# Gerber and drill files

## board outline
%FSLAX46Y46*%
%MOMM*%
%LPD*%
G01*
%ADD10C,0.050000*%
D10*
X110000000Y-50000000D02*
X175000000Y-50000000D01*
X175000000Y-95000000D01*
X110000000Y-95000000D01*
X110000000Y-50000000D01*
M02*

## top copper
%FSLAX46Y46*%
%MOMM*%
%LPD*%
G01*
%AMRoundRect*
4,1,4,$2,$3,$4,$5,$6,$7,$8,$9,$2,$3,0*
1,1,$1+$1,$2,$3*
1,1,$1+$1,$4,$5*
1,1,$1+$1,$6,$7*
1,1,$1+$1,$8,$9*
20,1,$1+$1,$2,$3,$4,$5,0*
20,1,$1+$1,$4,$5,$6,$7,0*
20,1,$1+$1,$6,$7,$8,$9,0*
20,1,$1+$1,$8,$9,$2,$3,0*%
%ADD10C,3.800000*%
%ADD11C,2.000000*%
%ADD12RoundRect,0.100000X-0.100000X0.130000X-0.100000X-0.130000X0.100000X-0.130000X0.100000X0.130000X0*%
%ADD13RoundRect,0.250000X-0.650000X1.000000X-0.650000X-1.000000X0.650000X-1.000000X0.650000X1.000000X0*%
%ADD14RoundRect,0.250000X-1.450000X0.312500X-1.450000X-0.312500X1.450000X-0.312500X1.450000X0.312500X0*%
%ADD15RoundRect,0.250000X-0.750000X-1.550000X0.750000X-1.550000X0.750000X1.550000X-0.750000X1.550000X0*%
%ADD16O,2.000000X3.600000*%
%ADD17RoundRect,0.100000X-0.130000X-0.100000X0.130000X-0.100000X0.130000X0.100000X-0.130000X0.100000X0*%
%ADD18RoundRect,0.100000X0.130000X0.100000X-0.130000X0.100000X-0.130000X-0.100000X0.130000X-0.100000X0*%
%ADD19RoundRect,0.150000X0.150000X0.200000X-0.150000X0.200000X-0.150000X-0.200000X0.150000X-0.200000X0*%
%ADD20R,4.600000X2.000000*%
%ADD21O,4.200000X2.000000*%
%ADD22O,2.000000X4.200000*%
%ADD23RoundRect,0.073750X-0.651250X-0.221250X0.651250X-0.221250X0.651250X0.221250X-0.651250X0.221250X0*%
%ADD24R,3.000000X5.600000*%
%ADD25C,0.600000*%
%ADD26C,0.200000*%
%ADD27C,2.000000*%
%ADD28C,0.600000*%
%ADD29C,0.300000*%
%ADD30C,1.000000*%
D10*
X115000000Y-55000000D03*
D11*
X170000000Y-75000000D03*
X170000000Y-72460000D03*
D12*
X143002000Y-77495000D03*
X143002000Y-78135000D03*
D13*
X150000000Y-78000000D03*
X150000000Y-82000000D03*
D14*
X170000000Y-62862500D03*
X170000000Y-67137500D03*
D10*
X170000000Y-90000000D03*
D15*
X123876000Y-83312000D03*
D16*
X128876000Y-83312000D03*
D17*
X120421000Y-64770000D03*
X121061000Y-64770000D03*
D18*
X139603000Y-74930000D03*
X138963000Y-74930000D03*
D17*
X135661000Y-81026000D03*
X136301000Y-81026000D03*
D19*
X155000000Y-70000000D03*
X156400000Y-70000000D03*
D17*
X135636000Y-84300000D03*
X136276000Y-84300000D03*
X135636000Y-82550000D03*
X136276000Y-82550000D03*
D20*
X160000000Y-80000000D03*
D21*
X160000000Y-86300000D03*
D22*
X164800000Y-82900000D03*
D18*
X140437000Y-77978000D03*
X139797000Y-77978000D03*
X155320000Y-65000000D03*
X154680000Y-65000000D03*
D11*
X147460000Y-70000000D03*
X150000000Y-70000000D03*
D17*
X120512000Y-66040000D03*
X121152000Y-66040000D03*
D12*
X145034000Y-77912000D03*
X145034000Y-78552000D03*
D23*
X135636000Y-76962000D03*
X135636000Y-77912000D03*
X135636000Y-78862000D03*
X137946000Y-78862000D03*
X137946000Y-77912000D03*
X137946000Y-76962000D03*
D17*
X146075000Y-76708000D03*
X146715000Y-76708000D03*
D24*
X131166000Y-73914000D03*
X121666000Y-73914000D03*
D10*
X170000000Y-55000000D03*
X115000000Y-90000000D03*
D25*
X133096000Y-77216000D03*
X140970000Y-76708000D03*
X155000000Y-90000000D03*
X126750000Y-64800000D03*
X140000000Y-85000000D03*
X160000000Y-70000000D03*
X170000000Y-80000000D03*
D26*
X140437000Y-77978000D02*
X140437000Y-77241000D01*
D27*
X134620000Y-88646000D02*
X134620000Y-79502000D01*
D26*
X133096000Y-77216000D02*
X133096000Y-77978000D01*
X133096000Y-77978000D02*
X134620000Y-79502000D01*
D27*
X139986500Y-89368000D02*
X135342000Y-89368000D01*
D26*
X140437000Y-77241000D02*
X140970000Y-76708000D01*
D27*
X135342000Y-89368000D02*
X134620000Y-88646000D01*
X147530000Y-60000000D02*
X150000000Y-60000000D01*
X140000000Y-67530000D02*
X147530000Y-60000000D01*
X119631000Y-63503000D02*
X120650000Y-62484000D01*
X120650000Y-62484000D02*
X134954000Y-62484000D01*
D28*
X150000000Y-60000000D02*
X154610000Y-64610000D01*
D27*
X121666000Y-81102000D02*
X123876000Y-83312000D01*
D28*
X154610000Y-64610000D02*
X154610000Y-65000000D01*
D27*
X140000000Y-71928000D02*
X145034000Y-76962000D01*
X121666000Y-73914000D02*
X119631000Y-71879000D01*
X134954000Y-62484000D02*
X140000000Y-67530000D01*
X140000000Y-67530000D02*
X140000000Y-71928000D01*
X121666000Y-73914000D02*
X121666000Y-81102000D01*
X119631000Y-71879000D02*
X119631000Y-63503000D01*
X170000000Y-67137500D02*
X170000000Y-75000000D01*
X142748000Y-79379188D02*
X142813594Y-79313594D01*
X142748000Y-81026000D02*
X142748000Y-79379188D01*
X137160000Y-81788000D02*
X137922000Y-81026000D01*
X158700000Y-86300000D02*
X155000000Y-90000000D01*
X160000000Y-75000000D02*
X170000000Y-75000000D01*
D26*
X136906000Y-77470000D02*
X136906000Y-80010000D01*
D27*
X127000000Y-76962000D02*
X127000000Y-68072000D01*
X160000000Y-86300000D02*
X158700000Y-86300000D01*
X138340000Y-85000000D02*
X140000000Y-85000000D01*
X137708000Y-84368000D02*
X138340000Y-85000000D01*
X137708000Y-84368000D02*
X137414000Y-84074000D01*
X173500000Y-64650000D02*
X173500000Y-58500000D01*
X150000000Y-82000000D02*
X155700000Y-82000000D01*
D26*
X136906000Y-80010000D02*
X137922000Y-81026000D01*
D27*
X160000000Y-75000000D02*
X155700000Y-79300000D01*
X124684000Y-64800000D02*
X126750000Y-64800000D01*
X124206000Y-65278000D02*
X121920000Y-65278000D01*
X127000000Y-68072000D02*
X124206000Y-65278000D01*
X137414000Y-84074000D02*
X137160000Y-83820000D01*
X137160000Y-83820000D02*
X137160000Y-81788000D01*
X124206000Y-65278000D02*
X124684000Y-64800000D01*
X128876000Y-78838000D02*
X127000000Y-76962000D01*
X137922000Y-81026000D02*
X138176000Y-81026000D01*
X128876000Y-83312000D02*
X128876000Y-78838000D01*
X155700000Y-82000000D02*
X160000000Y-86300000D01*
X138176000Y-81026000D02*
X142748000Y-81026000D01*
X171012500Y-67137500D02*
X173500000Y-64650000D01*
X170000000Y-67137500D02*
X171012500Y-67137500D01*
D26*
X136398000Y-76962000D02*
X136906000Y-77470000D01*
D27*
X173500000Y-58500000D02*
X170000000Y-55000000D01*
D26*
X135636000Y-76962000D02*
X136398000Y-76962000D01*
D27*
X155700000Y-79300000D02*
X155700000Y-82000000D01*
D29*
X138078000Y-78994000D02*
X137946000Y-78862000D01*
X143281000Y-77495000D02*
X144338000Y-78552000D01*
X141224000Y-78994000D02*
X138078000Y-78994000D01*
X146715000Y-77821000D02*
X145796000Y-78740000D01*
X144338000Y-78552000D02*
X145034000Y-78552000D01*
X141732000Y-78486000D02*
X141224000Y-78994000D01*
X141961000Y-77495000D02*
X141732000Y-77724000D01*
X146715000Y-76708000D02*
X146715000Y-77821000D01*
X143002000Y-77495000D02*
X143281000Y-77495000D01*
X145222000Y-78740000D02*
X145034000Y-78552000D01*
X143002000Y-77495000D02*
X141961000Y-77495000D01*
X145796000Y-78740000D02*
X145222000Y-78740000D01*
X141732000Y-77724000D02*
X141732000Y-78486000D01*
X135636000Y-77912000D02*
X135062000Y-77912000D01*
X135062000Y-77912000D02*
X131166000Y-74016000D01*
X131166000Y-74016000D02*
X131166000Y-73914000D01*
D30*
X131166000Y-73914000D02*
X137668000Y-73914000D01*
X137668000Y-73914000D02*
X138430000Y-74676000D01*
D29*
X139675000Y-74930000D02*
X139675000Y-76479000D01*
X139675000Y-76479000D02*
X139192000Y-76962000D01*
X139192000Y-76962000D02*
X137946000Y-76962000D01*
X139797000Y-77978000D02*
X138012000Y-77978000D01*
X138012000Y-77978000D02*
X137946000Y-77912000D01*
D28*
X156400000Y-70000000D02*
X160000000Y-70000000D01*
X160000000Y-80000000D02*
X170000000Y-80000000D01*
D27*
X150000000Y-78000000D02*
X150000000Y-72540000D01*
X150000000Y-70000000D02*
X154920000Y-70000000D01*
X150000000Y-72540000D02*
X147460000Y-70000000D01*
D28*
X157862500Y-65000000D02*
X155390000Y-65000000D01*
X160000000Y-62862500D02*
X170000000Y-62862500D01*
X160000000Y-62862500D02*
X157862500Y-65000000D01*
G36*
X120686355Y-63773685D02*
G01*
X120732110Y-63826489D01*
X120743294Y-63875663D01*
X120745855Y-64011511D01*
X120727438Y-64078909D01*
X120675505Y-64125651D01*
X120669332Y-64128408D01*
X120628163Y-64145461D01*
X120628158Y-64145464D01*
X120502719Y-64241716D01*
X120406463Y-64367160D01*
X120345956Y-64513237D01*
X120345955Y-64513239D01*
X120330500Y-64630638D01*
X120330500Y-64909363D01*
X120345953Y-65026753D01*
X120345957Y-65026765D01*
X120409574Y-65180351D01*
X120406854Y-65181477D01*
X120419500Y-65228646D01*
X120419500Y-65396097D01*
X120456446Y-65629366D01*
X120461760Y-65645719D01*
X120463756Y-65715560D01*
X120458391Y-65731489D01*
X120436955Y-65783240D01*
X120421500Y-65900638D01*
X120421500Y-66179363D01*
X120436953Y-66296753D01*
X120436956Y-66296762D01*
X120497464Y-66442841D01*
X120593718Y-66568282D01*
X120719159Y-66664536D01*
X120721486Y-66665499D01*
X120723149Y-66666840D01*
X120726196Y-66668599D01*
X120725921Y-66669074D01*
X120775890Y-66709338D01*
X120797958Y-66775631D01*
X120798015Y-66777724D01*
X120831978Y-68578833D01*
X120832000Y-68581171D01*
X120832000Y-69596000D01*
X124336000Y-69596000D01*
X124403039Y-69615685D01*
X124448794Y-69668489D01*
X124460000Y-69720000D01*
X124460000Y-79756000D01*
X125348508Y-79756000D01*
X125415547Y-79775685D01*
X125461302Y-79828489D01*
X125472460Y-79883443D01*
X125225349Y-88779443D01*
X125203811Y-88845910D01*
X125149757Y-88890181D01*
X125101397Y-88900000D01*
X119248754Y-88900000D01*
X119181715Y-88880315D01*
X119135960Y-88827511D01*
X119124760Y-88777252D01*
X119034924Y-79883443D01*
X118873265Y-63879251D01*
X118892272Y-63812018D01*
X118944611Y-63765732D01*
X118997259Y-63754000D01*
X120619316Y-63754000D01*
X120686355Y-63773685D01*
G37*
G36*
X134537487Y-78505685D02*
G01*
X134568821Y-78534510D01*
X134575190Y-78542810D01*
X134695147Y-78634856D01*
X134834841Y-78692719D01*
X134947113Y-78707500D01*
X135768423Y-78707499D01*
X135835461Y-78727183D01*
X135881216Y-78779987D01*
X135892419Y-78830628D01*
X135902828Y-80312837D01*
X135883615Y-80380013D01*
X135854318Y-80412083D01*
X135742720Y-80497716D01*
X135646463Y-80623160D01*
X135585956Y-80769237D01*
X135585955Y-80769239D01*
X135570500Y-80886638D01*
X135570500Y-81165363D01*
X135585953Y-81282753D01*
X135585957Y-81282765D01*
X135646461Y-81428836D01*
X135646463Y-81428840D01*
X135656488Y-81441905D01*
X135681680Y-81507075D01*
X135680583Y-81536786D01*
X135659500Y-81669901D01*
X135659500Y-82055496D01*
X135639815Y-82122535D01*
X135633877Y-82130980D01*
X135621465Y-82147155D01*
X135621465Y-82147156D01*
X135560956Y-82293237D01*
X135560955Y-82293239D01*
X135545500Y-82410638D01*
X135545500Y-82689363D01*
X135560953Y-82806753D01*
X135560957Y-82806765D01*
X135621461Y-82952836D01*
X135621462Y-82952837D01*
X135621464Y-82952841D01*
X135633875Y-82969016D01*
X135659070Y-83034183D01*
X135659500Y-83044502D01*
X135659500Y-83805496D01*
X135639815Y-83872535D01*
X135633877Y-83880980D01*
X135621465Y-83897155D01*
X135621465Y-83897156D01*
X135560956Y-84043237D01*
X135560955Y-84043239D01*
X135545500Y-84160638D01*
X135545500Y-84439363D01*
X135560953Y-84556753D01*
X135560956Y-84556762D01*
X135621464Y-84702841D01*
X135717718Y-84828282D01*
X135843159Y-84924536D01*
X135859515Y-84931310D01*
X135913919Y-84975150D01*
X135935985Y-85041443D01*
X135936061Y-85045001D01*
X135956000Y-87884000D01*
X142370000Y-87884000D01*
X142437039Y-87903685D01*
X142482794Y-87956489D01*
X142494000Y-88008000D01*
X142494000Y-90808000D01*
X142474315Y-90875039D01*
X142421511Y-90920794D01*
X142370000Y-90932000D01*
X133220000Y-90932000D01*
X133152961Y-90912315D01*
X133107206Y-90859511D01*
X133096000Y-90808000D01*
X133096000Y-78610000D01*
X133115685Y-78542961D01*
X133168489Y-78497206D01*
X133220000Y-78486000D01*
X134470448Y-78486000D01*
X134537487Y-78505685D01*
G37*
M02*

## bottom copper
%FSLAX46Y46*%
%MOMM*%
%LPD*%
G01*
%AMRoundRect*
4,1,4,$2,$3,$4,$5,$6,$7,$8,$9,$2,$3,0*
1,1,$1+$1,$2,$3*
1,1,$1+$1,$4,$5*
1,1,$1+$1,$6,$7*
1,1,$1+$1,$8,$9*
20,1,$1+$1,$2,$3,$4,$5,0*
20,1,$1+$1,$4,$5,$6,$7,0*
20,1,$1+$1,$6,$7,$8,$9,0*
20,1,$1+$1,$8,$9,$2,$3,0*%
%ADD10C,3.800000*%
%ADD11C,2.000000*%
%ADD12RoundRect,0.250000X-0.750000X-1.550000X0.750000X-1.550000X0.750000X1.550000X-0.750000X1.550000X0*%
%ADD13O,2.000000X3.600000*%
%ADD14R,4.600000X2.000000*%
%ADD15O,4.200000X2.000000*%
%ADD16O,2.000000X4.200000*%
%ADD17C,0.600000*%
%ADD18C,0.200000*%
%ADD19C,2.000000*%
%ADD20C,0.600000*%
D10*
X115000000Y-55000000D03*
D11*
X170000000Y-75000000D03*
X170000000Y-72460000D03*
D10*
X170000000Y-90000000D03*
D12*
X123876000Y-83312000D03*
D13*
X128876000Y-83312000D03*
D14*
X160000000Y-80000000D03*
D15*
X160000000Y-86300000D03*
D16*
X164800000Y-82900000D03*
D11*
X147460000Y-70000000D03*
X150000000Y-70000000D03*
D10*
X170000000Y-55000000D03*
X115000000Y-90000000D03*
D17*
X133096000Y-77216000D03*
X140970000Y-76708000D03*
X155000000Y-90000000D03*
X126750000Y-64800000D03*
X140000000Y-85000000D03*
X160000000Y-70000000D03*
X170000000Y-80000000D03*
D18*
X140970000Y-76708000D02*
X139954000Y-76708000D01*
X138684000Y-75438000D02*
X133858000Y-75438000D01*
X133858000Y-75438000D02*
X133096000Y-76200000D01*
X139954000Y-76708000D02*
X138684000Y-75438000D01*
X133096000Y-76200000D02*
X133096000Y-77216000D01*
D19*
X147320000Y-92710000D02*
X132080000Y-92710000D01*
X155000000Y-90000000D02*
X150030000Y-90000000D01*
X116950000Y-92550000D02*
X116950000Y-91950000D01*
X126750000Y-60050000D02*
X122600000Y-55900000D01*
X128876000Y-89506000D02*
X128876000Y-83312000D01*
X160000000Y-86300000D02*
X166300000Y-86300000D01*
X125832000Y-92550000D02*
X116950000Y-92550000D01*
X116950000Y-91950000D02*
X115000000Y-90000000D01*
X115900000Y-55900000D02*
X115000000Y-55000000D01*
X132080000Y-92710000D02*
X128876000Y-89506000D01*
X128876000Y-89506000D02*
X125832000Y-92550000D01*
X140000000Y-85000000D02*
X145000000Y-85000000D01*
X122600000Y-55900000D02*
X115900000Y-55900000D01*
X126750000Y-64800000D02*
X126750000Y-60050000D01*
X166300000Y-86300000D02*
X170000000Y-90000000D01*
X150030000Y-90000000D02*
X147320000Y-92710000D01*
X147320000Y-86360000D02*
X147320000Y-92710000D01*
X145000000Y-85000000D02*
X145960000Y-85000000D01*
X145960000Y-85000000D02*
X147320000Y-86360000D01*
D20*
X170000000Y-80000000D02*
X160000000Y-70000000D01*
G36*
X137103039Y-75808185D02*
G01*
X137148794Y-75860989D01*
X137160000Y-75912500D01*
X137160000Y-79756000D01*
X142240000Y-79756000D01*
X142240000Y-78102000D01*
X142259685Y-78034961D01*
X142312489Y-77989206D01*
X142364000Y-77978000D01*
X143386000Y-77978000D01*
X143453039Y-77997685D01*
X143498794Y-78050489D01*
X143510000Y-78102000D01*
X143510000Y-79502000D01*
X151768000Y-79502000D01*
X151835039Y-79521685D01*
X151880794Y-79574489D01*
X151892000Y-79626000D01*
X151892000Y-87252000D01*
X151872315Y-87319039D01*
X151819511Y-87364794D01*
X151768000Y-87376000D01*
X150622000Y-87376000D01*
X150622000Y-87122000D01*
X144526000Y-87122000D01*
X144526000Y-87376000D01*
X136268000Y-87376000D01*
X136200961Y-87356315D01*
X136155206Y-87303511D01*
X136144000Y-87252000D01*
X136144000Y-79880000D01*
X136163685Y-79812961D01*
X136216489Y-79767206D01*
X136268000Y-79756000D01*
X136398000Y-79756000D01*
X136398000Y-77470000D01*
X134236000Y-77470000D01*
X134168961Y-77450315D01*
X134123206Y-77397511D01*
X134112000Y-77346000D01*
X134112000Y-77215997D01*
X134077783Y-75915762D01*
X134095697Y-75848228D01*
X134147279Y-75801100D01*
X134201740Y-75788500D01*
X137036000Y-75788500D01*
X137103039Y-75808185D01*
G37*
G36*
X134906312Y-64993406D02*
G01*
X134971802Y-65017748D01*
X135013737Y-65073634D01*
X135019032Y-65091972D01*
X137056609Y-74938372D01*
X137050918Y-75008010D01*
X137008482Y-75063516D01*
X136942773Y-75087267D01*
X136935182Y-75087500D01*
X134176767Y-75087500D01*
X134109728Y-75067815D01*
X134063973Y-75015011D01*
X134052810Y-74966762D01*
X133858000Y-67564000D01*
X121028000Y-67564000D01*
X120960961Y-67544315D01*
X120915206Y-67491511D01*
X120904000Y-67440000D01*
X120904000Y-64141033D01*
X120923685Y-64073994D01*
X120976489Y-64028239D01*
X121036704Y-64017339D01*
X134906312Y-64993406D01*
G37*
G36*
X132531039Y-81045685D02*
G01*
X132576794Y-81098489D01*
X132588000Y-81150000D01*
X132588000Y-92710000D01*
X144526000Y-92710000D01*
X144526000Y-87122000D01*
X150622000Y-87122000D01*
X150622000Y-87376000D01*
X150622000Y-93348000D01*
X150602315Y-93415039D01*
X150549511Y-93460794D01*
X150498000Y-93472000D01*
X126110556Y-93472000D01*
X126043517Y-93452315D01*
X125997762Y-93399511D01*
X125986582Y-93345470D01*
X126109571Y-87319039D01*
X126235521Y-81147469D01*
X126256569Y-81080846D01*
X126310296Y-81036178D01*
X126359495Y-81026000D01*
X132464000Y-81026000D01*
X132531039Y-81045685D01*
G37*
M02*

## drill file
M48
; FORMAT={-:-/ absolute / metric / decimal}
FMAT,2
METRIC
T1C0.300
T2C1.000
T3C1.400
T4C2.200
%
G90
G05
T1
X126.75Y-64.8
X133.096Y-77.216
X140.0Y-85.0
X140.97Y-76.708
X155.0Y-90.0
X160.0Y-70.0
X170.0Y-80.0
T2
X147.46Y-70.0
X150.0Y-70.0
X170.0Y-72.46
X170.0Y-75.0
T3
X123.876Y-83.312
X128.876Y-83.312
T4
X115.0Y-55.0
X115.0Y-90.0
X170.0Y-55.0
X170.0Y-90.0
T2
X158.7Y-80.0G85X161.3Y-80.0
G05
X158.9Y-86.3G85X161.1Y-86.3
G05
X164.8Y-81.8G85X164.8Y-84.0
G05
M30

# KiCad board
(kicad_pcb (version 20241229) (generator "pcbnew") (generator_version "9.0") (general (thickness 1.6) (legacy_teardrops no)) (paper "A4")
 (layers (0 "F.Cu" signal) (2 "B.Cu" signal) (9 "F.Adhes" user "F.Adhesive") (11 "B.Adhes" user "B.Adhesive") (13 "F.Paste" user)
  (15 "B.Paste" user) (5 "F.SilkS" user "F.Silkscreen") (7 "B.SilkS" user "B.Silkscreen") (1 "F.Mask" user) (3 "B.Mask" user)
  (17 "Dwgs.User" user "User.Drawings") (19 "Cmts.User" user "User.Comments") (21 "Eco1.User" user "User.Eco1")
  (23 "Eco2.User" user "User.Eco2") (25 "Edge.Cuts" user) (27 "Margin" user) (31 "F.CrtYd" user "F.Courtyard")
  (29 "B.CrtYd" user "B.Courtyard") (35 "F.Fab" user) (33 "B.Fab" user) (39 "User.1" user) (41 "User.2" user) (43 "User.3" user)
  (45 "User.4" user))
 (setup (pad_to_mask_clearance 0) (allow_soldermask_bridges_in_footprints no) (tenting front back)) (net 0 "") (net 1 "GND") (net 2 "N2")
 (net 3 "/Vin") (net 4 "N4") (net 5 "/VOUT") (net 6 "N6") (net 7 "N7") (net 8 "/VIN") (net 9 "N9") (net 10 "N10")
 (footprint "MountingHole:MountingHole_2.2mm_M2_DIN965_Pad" (layer "F.Cu") (at 115 55)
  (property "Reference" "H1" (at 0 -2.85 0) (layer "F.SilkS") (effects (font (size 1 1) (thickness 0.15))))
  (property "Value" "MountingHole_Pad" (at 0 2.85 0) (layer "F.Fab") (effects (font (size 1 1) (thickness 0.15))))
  (pad "1" thru_hole circle (at 0 0) (size 3.8 3.8) (drill 2.2) (layers "*.Cu" "*.Mask") (remove_unused_layers no) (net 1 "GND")
   (zone_connect 2)))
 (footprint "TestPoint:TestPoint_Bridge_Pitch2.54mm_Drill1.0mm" (layer "F.Cu") (at 170 75 90)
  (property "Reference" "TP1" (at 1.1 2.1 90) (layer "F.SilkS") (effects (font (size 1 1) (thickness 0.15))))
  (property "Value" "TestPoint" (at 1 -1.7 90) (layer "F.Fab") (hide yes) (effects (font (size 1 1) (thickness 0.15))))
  (pad "1" thru_hole circle (at 0 0 90) (size 2 2) (drill 1) (layers "*.Cu" "*.Mask") (remove_unused_layers no) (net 1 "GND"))
  (pad "1" thru_hole circle (at 2.54 0 90) (size 2 2) (drill 1) (layers "*.Cu" "*.Mask") (remove_unused_layers no) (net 1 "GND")))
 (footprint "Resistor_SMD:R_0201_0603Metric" (layer "F.Cu") (at 143.002 77.815 -90)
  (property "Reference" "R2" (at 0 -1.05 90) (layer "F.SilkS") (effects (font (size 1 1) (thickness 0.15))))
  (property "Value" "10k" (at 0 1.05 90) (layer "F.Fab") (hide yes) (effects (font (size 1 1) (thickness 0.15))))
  (pad "" smd roundrect (at -0.345 0 270) (size 0.318 0.36) (layers "F.Paste") (roundrect_rratio 0.25))
  (pad "" smd roundrect (at 0.345 0 270) (size 0.318 0.36) (layers "F.Paste") (roundrect_rratio 0.25))
  (pad "1" smd roundrect (at -0.32 0 270) (size 0.46 0.4) (layers "F.Cu" "F.Mask") (roundrect_rratio 0.25) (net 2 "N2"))
  (pad "2" smd roundrect (at 0.32 0 270) (size 0.46 0.4) (layers "F.Cu" "F.Mask") (roundrect_rratio 0.25) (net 1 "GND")))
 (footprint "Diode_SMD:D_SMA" (layer "F.Cu") (at 150 80 -90)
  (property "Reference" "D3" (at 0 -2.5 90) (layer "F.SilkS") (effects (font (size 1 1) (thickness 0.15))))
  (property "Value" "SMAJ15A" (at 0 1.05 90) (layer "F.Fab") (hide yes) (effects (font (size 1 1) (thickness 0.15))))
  (pad "1" smd roundrect (at -2 0 270) (size 2.5 1.8) (layers "F.Cu" "F.Mask" "F.Paste") (roundrect_rratio 0.1388888889) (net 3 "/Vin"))
  (pad "2" smd roundrect (at 2 0 270) (size 2.5 1.8) (layers "F.Cu" "F.Mask" "F.Paste") (roundrect_rratio 0.1388888889) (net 1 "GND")))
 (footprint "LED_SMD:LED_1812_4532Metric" (layer "F.Cu") (at 170 65 -90)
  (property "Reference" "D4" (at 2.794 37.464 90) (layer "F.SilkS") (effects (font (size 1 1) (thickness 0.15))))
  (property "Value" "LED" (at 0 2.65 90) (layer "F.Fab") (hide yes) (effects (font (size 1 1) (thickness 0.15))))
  (pad "1" smd roundrect (at -2.1375 0 270) (size 1.125 3.4) (layers "F.Cu" "F.Mask" "F.Paste") (roundrect_rratio 0.222222) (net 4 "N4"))
  (pad "2" smd roundrect (at 2.1375 0 270) (size 1.125 3.4) (layers "F.Cu" "F.Mask" "F.Paste") (roundrect_rratio 0.222222) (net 1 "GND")))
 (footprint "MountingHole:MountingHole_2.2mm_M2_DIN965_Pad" (layer "F.Cu") (at 170 90)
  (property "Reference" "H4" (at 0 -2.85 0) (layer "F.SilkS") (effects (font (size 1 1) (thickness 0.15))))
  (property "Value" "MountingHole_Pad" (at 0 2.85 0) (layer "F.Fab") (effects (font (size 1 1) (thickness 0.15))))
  (pad "1" thru_hole circle (at 0 0) (size 3.8 3.8) (drill 2.2) (layers "*.Cu" "*.Mask") (remove_unused_layers no) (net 1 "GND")
   (zone_connect 2)))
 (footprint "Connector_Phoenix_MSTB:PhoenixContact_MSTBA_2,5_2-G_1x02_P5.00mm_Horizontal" (layer "F.Cu") (at 123.876 83.312)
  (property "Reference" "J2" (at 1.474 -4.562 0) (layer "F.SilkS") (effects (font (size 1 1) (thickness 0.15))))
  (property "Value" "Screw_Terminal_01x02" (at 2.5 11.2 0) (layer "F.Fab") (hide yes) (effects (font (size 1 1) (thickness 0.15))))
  (pad "1" thru_hole roundrect (at 0 0) (size 2 3.6) (drill 1.4) (layers "*.Cu" "*.Mask") (remove_unused_layers no) (roundrect_rratio 0.125)
   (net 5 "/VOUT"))
  (pad "2" thru_hole oval (at 5 0) (size 2 3.6) (drill 1.4) (layers "*.Cu" "*.Mask") (remove_unused_layers no) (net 1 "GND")))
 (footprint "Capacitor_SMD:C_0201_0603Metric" (layer "F.Cu") (at 120.741 64.77)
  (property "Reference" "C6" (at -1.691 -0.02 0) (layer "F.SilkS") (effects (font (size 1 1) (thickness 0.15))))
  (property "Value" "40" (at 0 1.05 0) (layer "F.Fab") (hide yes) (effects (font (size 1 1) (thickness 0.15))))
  (pad "" smd roundrect (at -0.345 0) (size 0.318 0.36) (layers "F.Paste") (roundrect_rratio 0.25))
  (pad "" smd roundrect (at 0.345 0) (size 0.318 0.36) (layers "F.Paste") (roundrect_rratio 0.25))
  (pad "1" smd roundrect (at -0.32 0) (size 0.46 0.4) (layers "F.Cu" "F.Mask") (roundrect_rratio 0.25) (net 5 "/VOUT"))
  (pad "2" smd roundrect (at 0.32 0) (size 0.46 0.4) (layers "F.Cu" "F.Mask") (roundrect_rratio 0.25) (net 1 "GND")))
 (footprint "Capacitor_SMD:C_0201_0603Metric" (layer "F.Cu") (at 139.283 74.93 180)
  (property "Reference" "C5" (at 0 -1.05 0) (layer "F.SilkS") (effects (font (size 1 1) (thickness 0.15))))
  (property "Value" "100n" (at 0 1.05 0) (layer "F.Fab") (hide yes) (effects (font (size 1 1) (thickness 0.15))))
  (pad "" smd roundrect (at -0.345 0 180) (size 0.318 0.36) (layers "F.Paste") (roundrect_rratio 0.25))
  (pad "" smd roundrect (at 0.345 0 180) (size 0.318 0.36) (layers "F.Paste") (roundrect_rratio 0.25))
  (pad "1" smd roundrect (at -0.32 0 180) (size 0.46 0.4) (layers "F.Cu" "F.Mask") (roundrect_rratio 0.25) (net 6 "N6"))
  (pad "2" smd roundrect (at 0.32 0 180) (size 0.46 0.4) (layers "F.Cu" "F.Mask") (roundrect_rratio 0.25) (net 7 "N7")))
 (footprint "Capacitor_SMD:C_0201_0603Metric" (layer "F.Cu") (at 135.981 81.026)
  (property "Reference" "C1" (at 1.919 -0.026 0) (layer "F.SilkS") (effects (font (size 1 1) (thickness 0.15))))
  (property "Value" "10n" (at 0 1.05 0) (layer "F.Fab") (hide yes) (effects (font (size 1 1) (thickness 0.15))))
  (pad "" smd roundrect (at -0.345 0) (size 0.318 0.36) (layers "F.Paste") (roundrect_rratio 0.25))
  (pad "" smd roundrect (at 0.345 0) (size 0.318 0.36) (layers "F.Paste") (roundrect_rratio 0.25))
  (pad "1" smd roundrect (at -0.32 0) (size 0.46 0.4) (layers "F.Cu" "F.Mask") (roundrect_rratio 0.25) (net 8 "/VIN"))
  (pad "2" smd roundrect (at 0.32 0) (size 0.46 0.4) (layers "F.Cu" "F.Mask") (roundrect_rratio 0.25) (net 1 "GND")))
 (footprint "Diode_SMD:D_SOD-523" (layer "F.Cu") (at 155.7 70)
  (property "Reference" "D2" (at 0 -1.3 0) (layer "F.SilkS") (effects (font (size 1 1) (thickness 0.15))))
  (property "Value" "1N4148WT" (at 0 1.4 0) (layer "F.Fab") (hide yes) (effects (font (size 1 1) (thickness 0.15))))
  (pad "1" smd roundrect (at -0.7 0 180) (size 0.6 0.7) (layers "F.Cu" "F.Mask" "F.Paste") (roundrect_rratio 0.25) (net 3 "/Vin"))
  (pad "2" smd roundrect (at 0.7 0 180) (size 0.6 0.7) (layers "F.Cu" "F.Mask" "F.Paste") (roundrect_rratio 0.25) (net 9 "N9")))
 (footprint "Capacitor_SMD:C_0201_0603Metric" (layer "F.Cu") (at 135.956 84.3)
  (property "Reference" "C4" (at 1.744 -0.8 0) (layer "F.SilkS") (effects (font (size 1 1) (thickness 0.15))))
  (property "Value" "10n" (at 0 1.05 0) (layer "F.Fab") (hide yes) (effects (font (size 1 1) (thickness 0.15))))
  (pad "" smd roundrect (at -0.345 0) (size 0.318 0.36) (layers "F.Paste") (roundrect_rratio 0.25))
  (pad "" smd roundrect (at 0.345 0) (size 0.318 0.36) (layers "F.Paste") (roundrect_rratio 0.25))
  (pad "1" smd roundrect (at -0.32 0) (size 0.46 0.4) (layers "F.Cu" "F.Mask") (roundrect_rratio 0.25) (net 8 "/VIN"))
  (pad "2" smd roundrect (at 0.32 0) (size 0.46 0.4) (layers "F.Cu" "F.Mask") (roundrect_rratio 0.25) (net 1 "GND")))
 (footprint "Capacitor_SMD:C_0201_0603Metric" (layer "F.Cu") (at 135.956 82.55)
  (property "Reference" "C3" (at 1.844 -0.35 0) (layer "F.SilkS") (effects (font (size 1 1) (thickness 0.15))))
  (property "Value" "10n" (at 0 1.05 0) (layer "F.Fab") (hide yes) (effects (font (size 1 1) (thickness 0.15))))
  (pad "" smd roundrect (at -0.345 0) (size 0.318 0.36) (layers "F.Paste") (roundrect_rratio 0.25))
  (pad "" smd roundrect (at 0.345 0) (size 0.318 0.36) (layers "F.Paste") (roundrect_rratio 0.25))
  (pad "1" smd roundrect (at -0.32 0) (size 0.46 0.4) (layers "F.Cu" "F.Mask") (roundrect_rratio 0.25) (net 8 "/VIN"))
  (pad "2" smd roundrect (at 0.32 0) (size 0.46 0.4) (layers "F.Cu" "F.Mask") (roundrect_rratio 0.25) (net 1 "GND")))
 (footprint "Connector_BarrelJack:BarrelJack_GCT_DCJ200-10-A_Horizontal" (layer "F.Cu") (at 160 80)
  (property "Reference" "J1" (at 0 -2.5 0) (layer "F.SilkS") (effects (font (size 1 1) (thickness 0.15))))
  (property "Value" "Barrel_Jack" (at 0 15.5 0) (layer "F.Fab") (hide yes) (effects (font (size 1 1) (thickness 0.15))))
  (pad "1" thru_hole rect (at 0 0) (size 4.6 2) (drill oval 3.6 1) (layers "*.Cu" "*.Mask") (remove_unused_layers no) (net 9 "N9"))
  (pad "2" thru_hole oval (at 0 6.3) (size 4.2 2) (drill oval 3.2 1) (layers "*.Cu" "*.Mask") (remove_unused_layers no) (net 1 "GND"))
  (pad "3" thru_hole oval (at 4.8 2.9) (size 2 4.2) (drill oval 1 3.2) (layers "*.Cu" "*.Mask") (remove_unused_layers no)))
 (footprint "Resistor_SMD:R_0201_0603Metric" (layer "F.Cu") (at 140.117 77.978 180)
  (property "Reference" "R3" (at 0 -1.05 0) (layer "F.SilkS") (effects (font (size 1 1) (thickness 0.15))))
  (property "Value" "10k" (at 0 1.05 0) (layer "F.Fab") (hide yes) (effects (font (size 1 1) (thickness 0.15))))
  (pad "" smd roundrect (at -0.345 0 180) (size 0.318 0.36) (layers "F.Paste") (roundrect_rratio 0.25))
  (pad "" smd roundrect (at 0.345 0 180) (size 0.318 0.36) (layers "F.Paste") (roundrect_rratio 0.25))
  (pad "1" smd roundrect (at -0.32 0 180) (size 0.46 0.4) (layers "F.Cu" "F.Mask") (roundrect_rratio 0.25) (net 8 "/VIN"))
  (pad "2" smd roundrect (at 0.32 0 180) (size 0.46 0.4) (layers "F.Cu" "F.Mask") (roundrect_rratio 0.25) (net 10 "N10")))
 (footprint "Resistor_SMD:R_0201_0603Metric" (layer "F.Cu") (at 155 65 180)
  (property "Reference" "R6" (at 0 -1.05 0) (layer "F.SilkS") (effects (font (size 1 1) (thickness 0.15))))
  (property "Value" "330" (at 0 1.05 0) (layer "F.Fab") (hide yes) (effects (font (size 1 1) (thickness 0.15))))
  (pad "" smd roundrect (at -0.345 0 180) (size 0.318 0.36) (layers "F.Paste") (roundrect_rratio 0.25))
  (pad "" smd roundrect (at 0.345 0 180) (size 0.318 0.36) (layers "F.Paste") (roundrect_rratio 0.25))
  (pad "1" smd roundrect (at -0.32 0 180) (size 0.46 0.4) (layers "F.Cu" "F.Mask") (roundrect_rratio 0.25) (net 4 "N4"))
  (pad "2" smd roundrect (at 0.32 0 180) (size 0.46 0.4) (layers "F.Cu" "F.Mask") (roundrect_rratio 0.25) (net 5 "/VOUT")))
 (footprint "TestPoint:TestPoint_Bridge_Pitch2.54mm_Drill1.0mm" (layer "F.Cu") (at 147.46 70)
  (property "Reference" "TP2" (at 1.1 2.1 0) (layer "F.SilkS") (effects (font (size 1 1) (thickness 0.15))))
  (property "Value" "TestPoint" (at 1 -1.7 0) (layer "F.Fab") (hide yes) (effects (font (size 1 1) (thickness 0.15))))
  (pad "1" thru_hole circle (at 0 0) (size 2 2) (drill 1) (layers "*.Cu" "*.Mask") (remove_unused_layers no) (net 3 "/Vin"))
  (pad "1" thru_hole circle (at 2.54 0) (size 2 2) (drill 1) (layers "*.Cu" "*.Mask") (remove_unused_layers no) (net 3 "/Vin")))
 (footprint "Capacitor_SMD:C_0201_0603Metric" (layer "F.Cu") (at 120.832 66.04)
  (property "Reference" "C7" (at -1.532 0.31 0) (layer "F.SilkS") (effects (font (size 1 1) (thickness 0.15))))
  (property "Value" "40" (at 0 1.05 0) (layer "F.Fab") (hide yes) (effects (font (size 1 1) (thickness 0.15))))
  (pad "" smd roundrect (at -0.345 0) (size 0.318 0.36) (layers "F.Paste") (roundrect_rratio 0.25))
  (pad "" smd roundrect (at 0.345 0) (size 0.318 0.36) (layers "F.Paste") (roundrect_rratio 0.25))
  (pad "1" smd roundrect (at -0.32 0) (size 0.46 0.4) (layers "F.Cu" "F.Mask") (roundrect_rratio 0.25) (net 5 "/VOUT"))
  (pad "2" smd roundrect (at 0.32 0) (size 0.46 0.4) (layers "F.Cu" "F.Mask") (roundrect_rratio 0.25) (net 1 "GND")))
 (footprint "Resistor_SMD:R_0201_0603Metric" (layer "F.Cu") (at 145.034 78.232 -90)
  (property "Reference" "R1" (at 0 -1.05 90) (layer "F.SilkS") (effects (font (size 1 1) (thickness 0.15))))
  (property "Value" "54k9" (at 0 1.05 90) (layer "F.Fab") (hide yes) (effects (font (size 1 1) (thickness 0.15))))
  (pad "" smd roundrect (at -0.345 0 270) (size 0.318 0.36) (layers "F.Paste") (roundrect_rratio 0.25))
  (pad "" smd roundrect (at 0.345 0 270) (size 0.318 0.36) (layers "F.Paste") (roundrect_rratio 0.25))
  (pad "1" smd roundrect (at -0.32 0 270) (size 0.46 0.4) (layers "F.Cu" "F.Mask") (roundrect_rratio 0.25) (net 5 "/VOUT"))
  (pad "2" smd roundrect (at 0.32 0 270) (size 0.46 0.4) (layers "F.Cu" "F.Mask") (roundrect_rratio 0.25) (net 2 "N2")))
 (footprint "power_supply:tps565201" (layer "F.Cu") (at 136.791 77.912)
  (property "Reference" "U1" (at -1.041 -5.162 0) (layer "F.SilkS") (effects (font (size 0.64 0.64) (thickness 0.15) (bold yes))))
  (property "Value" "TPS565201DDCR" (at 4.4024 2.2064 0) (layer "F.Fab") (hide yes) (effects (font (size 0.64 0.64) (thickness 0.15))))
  (pad "1" smd roundrect (at -1.155 -0.95) (size 1.45 0.59) (layers "F.Cu" "F.Mask" "F.Paste") (roundrect_rratio 0.125) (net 1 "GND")
   (solder_mask_margin 0.102))
  (pad "2" smd roundrect (at -1.155 0) (size 1.45 0.59) (layers "F.Cu" "F.Mask" "F.Paste") (roundrect_rratio 0.125) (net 7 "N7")
   (solder_mask_margin 0.102))
  (pad "3" smd roundrect (at -1.155 0.95) (size 1.45 0.59) (layers "F.Cu" "F.Mask" "F.Paste") (roundrect_rratio 0.125) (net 8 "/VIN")
   (solder_mask_margin 0.102))
  (pad "4" smd roundrect (at 1.155 0.95) (size 1.45 0.59) (layers "F.Cu" "F.Mask" "F.Paste") (roundrect_rratio 0.125) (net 2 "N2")
   (solder_mask_margin 0.102))
  (pad "5" smd roundrect (at 1.155 0) (size 1.45 0.59) (layers "F.Cu" "F.Mask" "F.Paste") (roundrect_rratio 0.125) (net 10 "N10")
   (solder_mask_margin 0.102))
  (pad "6" smd roundrect (at 1.155 -0.95) (size 1.45 0.59) (layers "F.Cu" "F.Mask" "F.Paste") (roundrect_rratio 0.125) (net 6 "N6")
   (solder_mask_margin 0.102)))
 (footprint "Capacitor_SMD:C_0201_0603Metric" (layer "F.Cu") (at 146.395 76.708)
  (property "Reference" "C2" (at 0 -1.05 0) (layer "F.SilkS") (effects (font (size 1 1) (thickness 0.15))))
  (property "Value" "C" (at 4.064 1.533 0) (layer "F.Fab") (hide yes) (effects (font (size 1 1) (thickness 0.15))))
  (pad "" smd roundrect (at -0.345 0) (size 0.318 0.36) (layers "F.Paste") (roundrect_rratio 0.25))
  (pad "" smd roundrect (at 0.345 0) (size 0.318 0.36) (layers "F.Paste") (roundrect_rratio 0.25))
  (pad "1" smd roundrect (at -0.32 0) (size 0.46 0.4) (layers "F.Cu" "F.Mask") (roundrect_rratio 0.25) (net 5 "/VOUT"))
  (pad "2" smd roundrect (at 0.32 0) (size 0.46 0.4) (layers "F.Cu" "F.Mask") (roundrect_rratio 0.25) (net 2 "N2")))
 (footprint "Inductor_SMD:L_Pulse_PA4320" (layer "F.Cu") (at 126.416 73.914 180)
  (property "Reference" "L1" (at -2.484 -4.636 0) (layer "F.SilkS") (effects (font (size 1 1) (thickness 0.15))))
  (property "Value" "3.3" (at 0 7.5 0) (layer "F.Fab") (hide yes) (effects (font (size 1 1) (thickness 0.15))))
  (pad "1" smd rect (at -4.75 0 270) (size 5.6 3) (layers "F.Cu" "F.Mask" "F.Paste") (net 7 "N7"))
  (pad "2" smd rect (at 4.75 0 270) (size 5.6 3) (layers "F.Cu" "F.Mask" "F.Paste") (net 5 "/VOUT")))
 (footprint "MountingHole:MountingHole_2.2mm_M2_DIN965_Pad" (layer "F.Cu") (at 170 55)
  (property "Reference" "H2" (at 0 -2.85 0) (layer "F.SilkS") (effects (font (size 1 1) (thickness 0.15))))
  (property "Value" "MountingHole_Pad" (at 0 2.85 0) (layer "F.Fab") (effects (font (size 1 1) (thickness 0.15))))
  (pad "1" thru_hole circle (at 0 0) (size 3.8 3.8) (drill 2.2) (layers "*.Cu" "*.Mask") (remove_unused_layers no) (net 1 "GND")
   (zone_connect 2)))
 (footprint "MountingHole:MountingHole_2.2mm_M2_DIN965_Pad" (layer "F.Cu") (at 115 90)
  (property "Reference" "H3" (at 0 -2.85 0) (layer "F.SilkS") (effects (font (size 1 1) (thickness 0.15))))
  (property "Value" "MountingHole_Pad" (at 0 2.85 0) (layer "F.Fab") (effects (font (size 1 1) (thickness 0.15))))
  (pad "1" thru_hole circle (at 0 0) (size 3.8 3.8) (drill 2.2) (layers "*.Cu" "*.Mask") (remove_unused_layers no) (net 1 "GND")
   (zone_connect 2)))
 (gr_rect (start 110 50) (end 175 95) (stroke (width 0.05) (type default)) (fill no) (layer "Edge.Cuts"))
 (segment (start 140.437 77.978) (end 140.437 77.241) (width 0.2) (layer "F.Cu") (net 8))
 (segment (start 134.62 88.646) (end 134.62 79.502) (width 2) (layer "F.Cu") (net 8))
 (segment (start 133.096 77.216) (end 133.096 77.978) (width 0.2) (layer "F.Cu") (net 8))
 (segment (start 133.096 77.978) (end 134.62 79.502) (width 0.2) (layer "F.Cu") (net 8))
 (segment (start 139.9865 89.368) (end 135.342 89.368) (width 2) (layer "F.Cu") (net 8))
 (segment (start 140.437 77.241) (end 140.97 76.708) (width 0.2) (layer "F.Cu") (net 8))
 (segment (start 135.342 89.368) (end 134.62 88.646) (width 2) (layer "F.Cu") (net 8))
 (via (at 133.096 77.216) (size 0.6) (drill 0.3) (layers "F.Cu" "B.Cu") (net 8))
 (via (at 140.97 76.708) (size 0.6) (drill 0.3) (layers "F.Cu" "B.Cu") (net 8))
 (segment (start 140.97 76.708) (end 139.954 76.708) (width 0.2) (layer "B.Cu") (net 8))
 (segment (start 138.684 75.438) (end 133.858 75.438) (width 0.2) (layer "B.Cu") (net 8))
 (segment (start 133.858 75.438) (end 133.096 76.2) (width 0.2) (layer "B.Cu") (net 8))
 (segment (start 139.954 76.708) (end 138.684 75.438) (width 0.2) (layer "B.Cu") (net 8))
 (segment (start 133.096 76.2) (end 133.096 77.216) (width 0.2) (layer "B.Cu") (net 8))
 (segment (start 147.53 60) (end 150 60) (width 2) (layer "F.Cu") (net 5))
 (segment (start 140 67.53) (end 147.53 60) (width 2) (layer "F.Cu") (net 5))
 (segment (start 119.631 63.503) (end 120.65 62.484) (width 2) (layer "F.Cu") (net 5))
 (segment (start 120.65 62.484) (end 134.954 62.484) (width 2) (layer "F.Cu") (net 5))
 (segment (start 150 60) (end 154.61 64.61) (width 0.6) (layer "F.Cu") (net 5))
 (segment (start 121.666 81.102) (end 123.876 83.312) (width 2) (layer "F.Cu") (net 5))
 (segment (start 154.61 64.61) (end 154.61 65) (width 0.6) (layer "F.Cu") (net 5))
 (segment (start 140 71.928) (end 145.034 76.962) (width 2) (layer "F.Cu") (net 5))
 (segment (start 121.666 73.914) (end 119.631 71.879) (width 2) (layer "F.Cu") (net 5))
 (segment (start 134.954 62.484) (end 140 67.53) (width 2) (layer "F.Cu") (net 5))
 (segment (start 140 67.53) (end 140 71.928) (width 2) (layer "F.Cu") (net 5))
 (segment (start 121.666 73.914) (end 121.666 81.102) (width 2) (layer "F.Cu") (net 5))
 (segment (start 119.631 71.879) (end 119.631 63.503) (width 2) (layer "F.Cu") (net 5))
 (segment (start 170 67.1375) (end 170 75) (width 2) (layer "F.Cu") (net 1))
 (segment (start 142.748 79.379188) (end 142.813594 79.313594) (width 2) (layer "F.Cu") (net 1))
 (segment (start 142.748 81.026) (end 142.748 79.379188) (width 2) (layer "F.Cu") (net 1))
 (segment (start 137.16 81.788) (end 137.922 81.026) (width 2) (layer "F.Cu") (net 1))
 (segment (start 158.7 86.3) (end 155 90) (width 2) (layer "F.Cu") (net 1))
 (segment (start 160 75) (end 170 75) (width 2) (layer "F.Cu") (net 1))
 (segment (start 136.906 77.47) (end 136.906 80.01) (width 0.2) (layer "F.Cu") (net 1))
 (segment (start 127 76.962) (end 127 68.072) (width 2) (layer "F.Cu") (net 1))
 (segment (start 160 86.3) (end 158.7 86.3) (width 2) (layer "F.Cu") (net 1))
 (segment (start 138.34 85) (end 140 85) (width 2) (layer "F.Cu") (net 1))
 (segment (start 137.708 84.368) (end 138.34 85) (width 2) (layer "F.Cu") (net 1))
 (segment (start 137.708 84.368) (end 137.414 84.074) (width 2) (layer "F.Cu") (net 1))
 (segment (start 173.5 64.65) (end 173.5 58.5) (width 2) (layer "F.Cu") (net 1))
 (segment (start 150 82) (end 155.7 82) (width 2) (layer "F.Cu") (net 1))
 (segment (start 136.906 80.01) (end 137.922 81.026) (width 0.2) (layer "F.Cu") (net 1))
 (segment (start 160 75) (end 155.7 79.3) (width 2) (layer "F.Cu") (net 1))
 (segment (start 124.684 64.8) (end 126.75 64.8) (width 2) (layer "F.Cu") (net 1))
 (segment (start 124.206 65.278) (end 121.92 65.278) (width 2) (layer "F.Cu") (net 1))
 (segment (start 127 68.072) (end 124.206 65.278) (width 2) (layer "F.Cu") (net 1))
 (segment (start 137.414 84.074) (end 137.16 83.82) (width 2) (layer "F.Cu") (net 1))
 (segment (start 137.16 83.82) (end 137.16 81.788) (width 2) (layer "F.Cu") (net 1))
 (segment (start 124.206 65.278) (end 124.684 64.8) (width 2) (layer "F.Cu") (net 1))
 (segment (start 128.876 78.838) (end 127 76.962) (width 2) (layer "F.Cu") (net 1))
 (segment (start 137.922 81.026) (end 138.176 81.026) (width 2) (layer "F.Cu") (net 1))
 (segment (start 128.876 83.312) (end 128.876 78.838) (width 2) (layer "F.Cu") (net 1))
 (segment (start 155.7 82) (end 160 86.3) (width 2) (layer "F.Cu") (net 1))
 (segment (start 138.176 81.026) (end 142.748 81.026) (width 2) (layer "F.Cu") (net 1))
 (segment (start 171.0125 67.1375) (end 173.5 64.65) (width 2) (layer "F.Cu") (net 1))
 (segment (start 170 67.1375) (end 171.0125 67.1375) (width 2) (layer "F.Cu") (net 1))
 (segment (start 136.398 76.962) (end 136.906 77.47) (width 0.2) (layer "F.Cu") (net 1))
 (segment (start 173.5 58.5) (end 170 55) (width 2) (layer "F.Cu") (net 1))
 (segment (start 135.636 76.962) (end 136.398 76.962) (width 0.2) (layer "F.Cu") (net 1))
 (segment (start 155.7 79.3) (end 155.7 82) (width 2) (layer "F.Cu") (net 1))
 (via (at 155 90) (size 0.6) (drill 0.3) (layers "F.Cu" "B.Cu") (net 1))
 (via (at 126.75 64.8) (size 0.6) (drill 0.3) (layers "F.Cu" "B.Cu") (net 1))
 (via (at 140 85) (size 0.6) (drill 0.3) (layers "F.Cu" "B.Cu") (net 1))
 (segment (start 147.32 92.71) (end 132.08 92.71) (width 2) (layer "B.Cu") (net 1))
 (segment (start 155 90) (end 150.03 90) (width 2) (layer "B.Cu") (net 1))
 (segment (start 116.95 92.55) (end 116.95 91.95) (width 2) (layer "B.Cu") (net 1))
 (segment (start 126.75 60.05) (end 122.6 55.9) (width 2) (layer "B.Cu") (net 1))
 (segment (start 128.876 89.506) (end 128.876 83.312) (width 2) (layer "B.Cu") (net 1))
 (segment (start 160 86.3) (end 166.3 86.3) (width 2) (layer "B.Cu") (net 1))
 (segment (start 125.832 92.55) (end 116.95 92.55) (width 2) (layer "B.Cu") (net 1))
 (segment (start 116.95 91.95) (end 115 90) (width 2) (layer "B.Cu") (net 1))
 (segment (start 115.9 55.9) (end 115 55) (width 2) (layer "B.Cu") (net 1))
 (segment (start 132.08 92.71) (end 128.876 89.506) (width 2) (layer "B.Cu") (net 1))
 (segment (start 128.876 89.506) (end 125.832 92.55) (width 2) (layer "B.Cu") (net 1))
 (segment (start 140 85) (end 145 85) (width 2) (layer "B.Cu") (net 1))
 (segment (start 122.6 55.9) (end 115.9 55.9) (width 2) (layer "B.Cu") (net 1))
 (segment (start 126.75 64.8) (end 126.75 60.05) (width 2) (layer "B.Cu") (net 1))
 (segment (start 166.3 86.3) (end 170 90) (width 2) (layer "B.Cu") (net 1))
 (segment (start 150.03 90) (end 147.32 92.71) (width 2) (layer "B.Cu") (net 1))
 (segment (start 147.32 86.36) (end 147.32 92.71) (width 2) (layer "B.Cu") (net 1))
 (segment (start 145 85) (end 145.96 85) (width 2) (layer "B.Cu") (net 1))
 (segment (start 145.96 85) (end 147.32 86.36) (width 2) (layer "B.Cu") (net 1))
 (segment (start 138.078 78.994) (end 137.946 78.862) (width 0.3) (layer "F.Cu") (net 2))
 (segment (start 143.281 77.495) (end 144.338 78.552) (width 0.3) (layer "F.Cu") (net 2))
 (segment (start 141.224 78.994) (end 138.078 78.994) (width 0.3) (layer "F.Cu") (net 2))
 (segment (start 146.715 77.821) (end 145.796 78.74) (width 0.3) (layer "F.Cu") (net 2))
 (segment (start 144.338 78.552) (end 145.034 78.552) (width 0.3) (layer "F.Cu") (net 2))
 (segment (start 141.732 78.486) (end 141.224 78.994) (width 0.3) (layer "F.Cu") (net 2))
 (segment (start 141.961 77.495) (end 141.732 77.724) (width 0.3) (layer "F.Cu") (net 2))
 (segment (start 146.715 76.708) (end 146.715 77.821) (width 0.3) (layer "F.Cu") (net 2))
 (segment (start 143.002 77.495) (end 143.281 77.495) (width 0.3) (layer "F.Cu") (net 2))
 (segment (start 145.222 78.74) (end 145.034 78.552) (width 0.3) (layer "F.Cu") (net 2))
 (segment (start 143.002 77.495) (end 141.961 77.495) (width 0.3) (layer "F.Cu") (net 2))
 (segment (start 145.796 78.74) (end 145.222 78.74) (width 0.3) (layer "F.Cu") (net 2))
 (segment (start 141.732 77.724) (end 141.732 78.486) (width 0.3) (layer "F.Cu") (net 2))
 (segment (start 135.636 77.912) (end 135.062 77.912) (width 0.3) (layer "F.Cu") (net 7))
 (segment (start 135.062 77.912) (end 131.166 74.016) (width 0.3) (layer "F.Cu") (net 7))
 (segment (start 131.166 74.016) (end 131.166 73.914) (width 0.3) (layer "F.Cu") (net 7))
 (segment (start 131.166 73.914) (end 137.668 73.914) (width 1) (layer "F.Cu") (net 7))
 (segment (start 137.668 73.914) (end 138.43 74.676) (width 1) (layer "F.Cu") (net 7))
 (segment (start 139.675 74.93) (end 139.675 76.479) (width 0.3) (layer "F.Cu") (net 6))
 (segment (start 139.675 76.479) (end 139.192 76.962) (width 0.3) (layer "F.Cu") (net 6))
 (segment (start 139.192 76.962) (end 137.946 76.962) (width 0.3) (layer "F.Cu") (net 6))
 (segment (start 139.797 77.978) (end 138.012 77.978) (width 0.3) (layer "F.Cu") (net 10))
 (segment (start 138.012 77.978) (end 137.946 77.912) (width 0.3) (layer "F.Cu") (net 10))
 (segment (start 156.4 70) (end 160 70) (width 0.6) (layer "F.Cu") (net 9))
 (segment (start 160 80) (end 170 80) (width 0.6) (layer "F.Cu") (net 9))
 (via (at 160 70) (size 0.6) (drill 0.3) (layers "F.Cu" "B.Cu") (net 9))
 (via (at 170 80) (size 0.6) (drill 0.3) (layers "F.Cu" "B.Cu") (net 9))
 (segment (start 170 80) (end 160 70) (width 0.6) (layer "B.Cu") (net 9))
 (segment (start 150 78) (end 150 72.54) (width 2) (layer "F.Cu") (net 3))
 (segment (start 150 70) (end 154.92 70) (width 2) (layer "F.Cu") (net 3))
 (segment (start 150 72.54) (end 147.46 70) (width 2) (layer "F.Cu") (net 3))
 (segment (start 157.8625 65) (end 155.39 65) (width 0.6) (layer "F.Cu") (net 4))
 (segment (start 160 62.8625) (end 170 62.8625) (width 0.6) (layer "F.Cu") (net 4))
 (segment (start 160 62.8625) (end 157.8625 65) (width 0.6) (layer "F.Cu") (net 4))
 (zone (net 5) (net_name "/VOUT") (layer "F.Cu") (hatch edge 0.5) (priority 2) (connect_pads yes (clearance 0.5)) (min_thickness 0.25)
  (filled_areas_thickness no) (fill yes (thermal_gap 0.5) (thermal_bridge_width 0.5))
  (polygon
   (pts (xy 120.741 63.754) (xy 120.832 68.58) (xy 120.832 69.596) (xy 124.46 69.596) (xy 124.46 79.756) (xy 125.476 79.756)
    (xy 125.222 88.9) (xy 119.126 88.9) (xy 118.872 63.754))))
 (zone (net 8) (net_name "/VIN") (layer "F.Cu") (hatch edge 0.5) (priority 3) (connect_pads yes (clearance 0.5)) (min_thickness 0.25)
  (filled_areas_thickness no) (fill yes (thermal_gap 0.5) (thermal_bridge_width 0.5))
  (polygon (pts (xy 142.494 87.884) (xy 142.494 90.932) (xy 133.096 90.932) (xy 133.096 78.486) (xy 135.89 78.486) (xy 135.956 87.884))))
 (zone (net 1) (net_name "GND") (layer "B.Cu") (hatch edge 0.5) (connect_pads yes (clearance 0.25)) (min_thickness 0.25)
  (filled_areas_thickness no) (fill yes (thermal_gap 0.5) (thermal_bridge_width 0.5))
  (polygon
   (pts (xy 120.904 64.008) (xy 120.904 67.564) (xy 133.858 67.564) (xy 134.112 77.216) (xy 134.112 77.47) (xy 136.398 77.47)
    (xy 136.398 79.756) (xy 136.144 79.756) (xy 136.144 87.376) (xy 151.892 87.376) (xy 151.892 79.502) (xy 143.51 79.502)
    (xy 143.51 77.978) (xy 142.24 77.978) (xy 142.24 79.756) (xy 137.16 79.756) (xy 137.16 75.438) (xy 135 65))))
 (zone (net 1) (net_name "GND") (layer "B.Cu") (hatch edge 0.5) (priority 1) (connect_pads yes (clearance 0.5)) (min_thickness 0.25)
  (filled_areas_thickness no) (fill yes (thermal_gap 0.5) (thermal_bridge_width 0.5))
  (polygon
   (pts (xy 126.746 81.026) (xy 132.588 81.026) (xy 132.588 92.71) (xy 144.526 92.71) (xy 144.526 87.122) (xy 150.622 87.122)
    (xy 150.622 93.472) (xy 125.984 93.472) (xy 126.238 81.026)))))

